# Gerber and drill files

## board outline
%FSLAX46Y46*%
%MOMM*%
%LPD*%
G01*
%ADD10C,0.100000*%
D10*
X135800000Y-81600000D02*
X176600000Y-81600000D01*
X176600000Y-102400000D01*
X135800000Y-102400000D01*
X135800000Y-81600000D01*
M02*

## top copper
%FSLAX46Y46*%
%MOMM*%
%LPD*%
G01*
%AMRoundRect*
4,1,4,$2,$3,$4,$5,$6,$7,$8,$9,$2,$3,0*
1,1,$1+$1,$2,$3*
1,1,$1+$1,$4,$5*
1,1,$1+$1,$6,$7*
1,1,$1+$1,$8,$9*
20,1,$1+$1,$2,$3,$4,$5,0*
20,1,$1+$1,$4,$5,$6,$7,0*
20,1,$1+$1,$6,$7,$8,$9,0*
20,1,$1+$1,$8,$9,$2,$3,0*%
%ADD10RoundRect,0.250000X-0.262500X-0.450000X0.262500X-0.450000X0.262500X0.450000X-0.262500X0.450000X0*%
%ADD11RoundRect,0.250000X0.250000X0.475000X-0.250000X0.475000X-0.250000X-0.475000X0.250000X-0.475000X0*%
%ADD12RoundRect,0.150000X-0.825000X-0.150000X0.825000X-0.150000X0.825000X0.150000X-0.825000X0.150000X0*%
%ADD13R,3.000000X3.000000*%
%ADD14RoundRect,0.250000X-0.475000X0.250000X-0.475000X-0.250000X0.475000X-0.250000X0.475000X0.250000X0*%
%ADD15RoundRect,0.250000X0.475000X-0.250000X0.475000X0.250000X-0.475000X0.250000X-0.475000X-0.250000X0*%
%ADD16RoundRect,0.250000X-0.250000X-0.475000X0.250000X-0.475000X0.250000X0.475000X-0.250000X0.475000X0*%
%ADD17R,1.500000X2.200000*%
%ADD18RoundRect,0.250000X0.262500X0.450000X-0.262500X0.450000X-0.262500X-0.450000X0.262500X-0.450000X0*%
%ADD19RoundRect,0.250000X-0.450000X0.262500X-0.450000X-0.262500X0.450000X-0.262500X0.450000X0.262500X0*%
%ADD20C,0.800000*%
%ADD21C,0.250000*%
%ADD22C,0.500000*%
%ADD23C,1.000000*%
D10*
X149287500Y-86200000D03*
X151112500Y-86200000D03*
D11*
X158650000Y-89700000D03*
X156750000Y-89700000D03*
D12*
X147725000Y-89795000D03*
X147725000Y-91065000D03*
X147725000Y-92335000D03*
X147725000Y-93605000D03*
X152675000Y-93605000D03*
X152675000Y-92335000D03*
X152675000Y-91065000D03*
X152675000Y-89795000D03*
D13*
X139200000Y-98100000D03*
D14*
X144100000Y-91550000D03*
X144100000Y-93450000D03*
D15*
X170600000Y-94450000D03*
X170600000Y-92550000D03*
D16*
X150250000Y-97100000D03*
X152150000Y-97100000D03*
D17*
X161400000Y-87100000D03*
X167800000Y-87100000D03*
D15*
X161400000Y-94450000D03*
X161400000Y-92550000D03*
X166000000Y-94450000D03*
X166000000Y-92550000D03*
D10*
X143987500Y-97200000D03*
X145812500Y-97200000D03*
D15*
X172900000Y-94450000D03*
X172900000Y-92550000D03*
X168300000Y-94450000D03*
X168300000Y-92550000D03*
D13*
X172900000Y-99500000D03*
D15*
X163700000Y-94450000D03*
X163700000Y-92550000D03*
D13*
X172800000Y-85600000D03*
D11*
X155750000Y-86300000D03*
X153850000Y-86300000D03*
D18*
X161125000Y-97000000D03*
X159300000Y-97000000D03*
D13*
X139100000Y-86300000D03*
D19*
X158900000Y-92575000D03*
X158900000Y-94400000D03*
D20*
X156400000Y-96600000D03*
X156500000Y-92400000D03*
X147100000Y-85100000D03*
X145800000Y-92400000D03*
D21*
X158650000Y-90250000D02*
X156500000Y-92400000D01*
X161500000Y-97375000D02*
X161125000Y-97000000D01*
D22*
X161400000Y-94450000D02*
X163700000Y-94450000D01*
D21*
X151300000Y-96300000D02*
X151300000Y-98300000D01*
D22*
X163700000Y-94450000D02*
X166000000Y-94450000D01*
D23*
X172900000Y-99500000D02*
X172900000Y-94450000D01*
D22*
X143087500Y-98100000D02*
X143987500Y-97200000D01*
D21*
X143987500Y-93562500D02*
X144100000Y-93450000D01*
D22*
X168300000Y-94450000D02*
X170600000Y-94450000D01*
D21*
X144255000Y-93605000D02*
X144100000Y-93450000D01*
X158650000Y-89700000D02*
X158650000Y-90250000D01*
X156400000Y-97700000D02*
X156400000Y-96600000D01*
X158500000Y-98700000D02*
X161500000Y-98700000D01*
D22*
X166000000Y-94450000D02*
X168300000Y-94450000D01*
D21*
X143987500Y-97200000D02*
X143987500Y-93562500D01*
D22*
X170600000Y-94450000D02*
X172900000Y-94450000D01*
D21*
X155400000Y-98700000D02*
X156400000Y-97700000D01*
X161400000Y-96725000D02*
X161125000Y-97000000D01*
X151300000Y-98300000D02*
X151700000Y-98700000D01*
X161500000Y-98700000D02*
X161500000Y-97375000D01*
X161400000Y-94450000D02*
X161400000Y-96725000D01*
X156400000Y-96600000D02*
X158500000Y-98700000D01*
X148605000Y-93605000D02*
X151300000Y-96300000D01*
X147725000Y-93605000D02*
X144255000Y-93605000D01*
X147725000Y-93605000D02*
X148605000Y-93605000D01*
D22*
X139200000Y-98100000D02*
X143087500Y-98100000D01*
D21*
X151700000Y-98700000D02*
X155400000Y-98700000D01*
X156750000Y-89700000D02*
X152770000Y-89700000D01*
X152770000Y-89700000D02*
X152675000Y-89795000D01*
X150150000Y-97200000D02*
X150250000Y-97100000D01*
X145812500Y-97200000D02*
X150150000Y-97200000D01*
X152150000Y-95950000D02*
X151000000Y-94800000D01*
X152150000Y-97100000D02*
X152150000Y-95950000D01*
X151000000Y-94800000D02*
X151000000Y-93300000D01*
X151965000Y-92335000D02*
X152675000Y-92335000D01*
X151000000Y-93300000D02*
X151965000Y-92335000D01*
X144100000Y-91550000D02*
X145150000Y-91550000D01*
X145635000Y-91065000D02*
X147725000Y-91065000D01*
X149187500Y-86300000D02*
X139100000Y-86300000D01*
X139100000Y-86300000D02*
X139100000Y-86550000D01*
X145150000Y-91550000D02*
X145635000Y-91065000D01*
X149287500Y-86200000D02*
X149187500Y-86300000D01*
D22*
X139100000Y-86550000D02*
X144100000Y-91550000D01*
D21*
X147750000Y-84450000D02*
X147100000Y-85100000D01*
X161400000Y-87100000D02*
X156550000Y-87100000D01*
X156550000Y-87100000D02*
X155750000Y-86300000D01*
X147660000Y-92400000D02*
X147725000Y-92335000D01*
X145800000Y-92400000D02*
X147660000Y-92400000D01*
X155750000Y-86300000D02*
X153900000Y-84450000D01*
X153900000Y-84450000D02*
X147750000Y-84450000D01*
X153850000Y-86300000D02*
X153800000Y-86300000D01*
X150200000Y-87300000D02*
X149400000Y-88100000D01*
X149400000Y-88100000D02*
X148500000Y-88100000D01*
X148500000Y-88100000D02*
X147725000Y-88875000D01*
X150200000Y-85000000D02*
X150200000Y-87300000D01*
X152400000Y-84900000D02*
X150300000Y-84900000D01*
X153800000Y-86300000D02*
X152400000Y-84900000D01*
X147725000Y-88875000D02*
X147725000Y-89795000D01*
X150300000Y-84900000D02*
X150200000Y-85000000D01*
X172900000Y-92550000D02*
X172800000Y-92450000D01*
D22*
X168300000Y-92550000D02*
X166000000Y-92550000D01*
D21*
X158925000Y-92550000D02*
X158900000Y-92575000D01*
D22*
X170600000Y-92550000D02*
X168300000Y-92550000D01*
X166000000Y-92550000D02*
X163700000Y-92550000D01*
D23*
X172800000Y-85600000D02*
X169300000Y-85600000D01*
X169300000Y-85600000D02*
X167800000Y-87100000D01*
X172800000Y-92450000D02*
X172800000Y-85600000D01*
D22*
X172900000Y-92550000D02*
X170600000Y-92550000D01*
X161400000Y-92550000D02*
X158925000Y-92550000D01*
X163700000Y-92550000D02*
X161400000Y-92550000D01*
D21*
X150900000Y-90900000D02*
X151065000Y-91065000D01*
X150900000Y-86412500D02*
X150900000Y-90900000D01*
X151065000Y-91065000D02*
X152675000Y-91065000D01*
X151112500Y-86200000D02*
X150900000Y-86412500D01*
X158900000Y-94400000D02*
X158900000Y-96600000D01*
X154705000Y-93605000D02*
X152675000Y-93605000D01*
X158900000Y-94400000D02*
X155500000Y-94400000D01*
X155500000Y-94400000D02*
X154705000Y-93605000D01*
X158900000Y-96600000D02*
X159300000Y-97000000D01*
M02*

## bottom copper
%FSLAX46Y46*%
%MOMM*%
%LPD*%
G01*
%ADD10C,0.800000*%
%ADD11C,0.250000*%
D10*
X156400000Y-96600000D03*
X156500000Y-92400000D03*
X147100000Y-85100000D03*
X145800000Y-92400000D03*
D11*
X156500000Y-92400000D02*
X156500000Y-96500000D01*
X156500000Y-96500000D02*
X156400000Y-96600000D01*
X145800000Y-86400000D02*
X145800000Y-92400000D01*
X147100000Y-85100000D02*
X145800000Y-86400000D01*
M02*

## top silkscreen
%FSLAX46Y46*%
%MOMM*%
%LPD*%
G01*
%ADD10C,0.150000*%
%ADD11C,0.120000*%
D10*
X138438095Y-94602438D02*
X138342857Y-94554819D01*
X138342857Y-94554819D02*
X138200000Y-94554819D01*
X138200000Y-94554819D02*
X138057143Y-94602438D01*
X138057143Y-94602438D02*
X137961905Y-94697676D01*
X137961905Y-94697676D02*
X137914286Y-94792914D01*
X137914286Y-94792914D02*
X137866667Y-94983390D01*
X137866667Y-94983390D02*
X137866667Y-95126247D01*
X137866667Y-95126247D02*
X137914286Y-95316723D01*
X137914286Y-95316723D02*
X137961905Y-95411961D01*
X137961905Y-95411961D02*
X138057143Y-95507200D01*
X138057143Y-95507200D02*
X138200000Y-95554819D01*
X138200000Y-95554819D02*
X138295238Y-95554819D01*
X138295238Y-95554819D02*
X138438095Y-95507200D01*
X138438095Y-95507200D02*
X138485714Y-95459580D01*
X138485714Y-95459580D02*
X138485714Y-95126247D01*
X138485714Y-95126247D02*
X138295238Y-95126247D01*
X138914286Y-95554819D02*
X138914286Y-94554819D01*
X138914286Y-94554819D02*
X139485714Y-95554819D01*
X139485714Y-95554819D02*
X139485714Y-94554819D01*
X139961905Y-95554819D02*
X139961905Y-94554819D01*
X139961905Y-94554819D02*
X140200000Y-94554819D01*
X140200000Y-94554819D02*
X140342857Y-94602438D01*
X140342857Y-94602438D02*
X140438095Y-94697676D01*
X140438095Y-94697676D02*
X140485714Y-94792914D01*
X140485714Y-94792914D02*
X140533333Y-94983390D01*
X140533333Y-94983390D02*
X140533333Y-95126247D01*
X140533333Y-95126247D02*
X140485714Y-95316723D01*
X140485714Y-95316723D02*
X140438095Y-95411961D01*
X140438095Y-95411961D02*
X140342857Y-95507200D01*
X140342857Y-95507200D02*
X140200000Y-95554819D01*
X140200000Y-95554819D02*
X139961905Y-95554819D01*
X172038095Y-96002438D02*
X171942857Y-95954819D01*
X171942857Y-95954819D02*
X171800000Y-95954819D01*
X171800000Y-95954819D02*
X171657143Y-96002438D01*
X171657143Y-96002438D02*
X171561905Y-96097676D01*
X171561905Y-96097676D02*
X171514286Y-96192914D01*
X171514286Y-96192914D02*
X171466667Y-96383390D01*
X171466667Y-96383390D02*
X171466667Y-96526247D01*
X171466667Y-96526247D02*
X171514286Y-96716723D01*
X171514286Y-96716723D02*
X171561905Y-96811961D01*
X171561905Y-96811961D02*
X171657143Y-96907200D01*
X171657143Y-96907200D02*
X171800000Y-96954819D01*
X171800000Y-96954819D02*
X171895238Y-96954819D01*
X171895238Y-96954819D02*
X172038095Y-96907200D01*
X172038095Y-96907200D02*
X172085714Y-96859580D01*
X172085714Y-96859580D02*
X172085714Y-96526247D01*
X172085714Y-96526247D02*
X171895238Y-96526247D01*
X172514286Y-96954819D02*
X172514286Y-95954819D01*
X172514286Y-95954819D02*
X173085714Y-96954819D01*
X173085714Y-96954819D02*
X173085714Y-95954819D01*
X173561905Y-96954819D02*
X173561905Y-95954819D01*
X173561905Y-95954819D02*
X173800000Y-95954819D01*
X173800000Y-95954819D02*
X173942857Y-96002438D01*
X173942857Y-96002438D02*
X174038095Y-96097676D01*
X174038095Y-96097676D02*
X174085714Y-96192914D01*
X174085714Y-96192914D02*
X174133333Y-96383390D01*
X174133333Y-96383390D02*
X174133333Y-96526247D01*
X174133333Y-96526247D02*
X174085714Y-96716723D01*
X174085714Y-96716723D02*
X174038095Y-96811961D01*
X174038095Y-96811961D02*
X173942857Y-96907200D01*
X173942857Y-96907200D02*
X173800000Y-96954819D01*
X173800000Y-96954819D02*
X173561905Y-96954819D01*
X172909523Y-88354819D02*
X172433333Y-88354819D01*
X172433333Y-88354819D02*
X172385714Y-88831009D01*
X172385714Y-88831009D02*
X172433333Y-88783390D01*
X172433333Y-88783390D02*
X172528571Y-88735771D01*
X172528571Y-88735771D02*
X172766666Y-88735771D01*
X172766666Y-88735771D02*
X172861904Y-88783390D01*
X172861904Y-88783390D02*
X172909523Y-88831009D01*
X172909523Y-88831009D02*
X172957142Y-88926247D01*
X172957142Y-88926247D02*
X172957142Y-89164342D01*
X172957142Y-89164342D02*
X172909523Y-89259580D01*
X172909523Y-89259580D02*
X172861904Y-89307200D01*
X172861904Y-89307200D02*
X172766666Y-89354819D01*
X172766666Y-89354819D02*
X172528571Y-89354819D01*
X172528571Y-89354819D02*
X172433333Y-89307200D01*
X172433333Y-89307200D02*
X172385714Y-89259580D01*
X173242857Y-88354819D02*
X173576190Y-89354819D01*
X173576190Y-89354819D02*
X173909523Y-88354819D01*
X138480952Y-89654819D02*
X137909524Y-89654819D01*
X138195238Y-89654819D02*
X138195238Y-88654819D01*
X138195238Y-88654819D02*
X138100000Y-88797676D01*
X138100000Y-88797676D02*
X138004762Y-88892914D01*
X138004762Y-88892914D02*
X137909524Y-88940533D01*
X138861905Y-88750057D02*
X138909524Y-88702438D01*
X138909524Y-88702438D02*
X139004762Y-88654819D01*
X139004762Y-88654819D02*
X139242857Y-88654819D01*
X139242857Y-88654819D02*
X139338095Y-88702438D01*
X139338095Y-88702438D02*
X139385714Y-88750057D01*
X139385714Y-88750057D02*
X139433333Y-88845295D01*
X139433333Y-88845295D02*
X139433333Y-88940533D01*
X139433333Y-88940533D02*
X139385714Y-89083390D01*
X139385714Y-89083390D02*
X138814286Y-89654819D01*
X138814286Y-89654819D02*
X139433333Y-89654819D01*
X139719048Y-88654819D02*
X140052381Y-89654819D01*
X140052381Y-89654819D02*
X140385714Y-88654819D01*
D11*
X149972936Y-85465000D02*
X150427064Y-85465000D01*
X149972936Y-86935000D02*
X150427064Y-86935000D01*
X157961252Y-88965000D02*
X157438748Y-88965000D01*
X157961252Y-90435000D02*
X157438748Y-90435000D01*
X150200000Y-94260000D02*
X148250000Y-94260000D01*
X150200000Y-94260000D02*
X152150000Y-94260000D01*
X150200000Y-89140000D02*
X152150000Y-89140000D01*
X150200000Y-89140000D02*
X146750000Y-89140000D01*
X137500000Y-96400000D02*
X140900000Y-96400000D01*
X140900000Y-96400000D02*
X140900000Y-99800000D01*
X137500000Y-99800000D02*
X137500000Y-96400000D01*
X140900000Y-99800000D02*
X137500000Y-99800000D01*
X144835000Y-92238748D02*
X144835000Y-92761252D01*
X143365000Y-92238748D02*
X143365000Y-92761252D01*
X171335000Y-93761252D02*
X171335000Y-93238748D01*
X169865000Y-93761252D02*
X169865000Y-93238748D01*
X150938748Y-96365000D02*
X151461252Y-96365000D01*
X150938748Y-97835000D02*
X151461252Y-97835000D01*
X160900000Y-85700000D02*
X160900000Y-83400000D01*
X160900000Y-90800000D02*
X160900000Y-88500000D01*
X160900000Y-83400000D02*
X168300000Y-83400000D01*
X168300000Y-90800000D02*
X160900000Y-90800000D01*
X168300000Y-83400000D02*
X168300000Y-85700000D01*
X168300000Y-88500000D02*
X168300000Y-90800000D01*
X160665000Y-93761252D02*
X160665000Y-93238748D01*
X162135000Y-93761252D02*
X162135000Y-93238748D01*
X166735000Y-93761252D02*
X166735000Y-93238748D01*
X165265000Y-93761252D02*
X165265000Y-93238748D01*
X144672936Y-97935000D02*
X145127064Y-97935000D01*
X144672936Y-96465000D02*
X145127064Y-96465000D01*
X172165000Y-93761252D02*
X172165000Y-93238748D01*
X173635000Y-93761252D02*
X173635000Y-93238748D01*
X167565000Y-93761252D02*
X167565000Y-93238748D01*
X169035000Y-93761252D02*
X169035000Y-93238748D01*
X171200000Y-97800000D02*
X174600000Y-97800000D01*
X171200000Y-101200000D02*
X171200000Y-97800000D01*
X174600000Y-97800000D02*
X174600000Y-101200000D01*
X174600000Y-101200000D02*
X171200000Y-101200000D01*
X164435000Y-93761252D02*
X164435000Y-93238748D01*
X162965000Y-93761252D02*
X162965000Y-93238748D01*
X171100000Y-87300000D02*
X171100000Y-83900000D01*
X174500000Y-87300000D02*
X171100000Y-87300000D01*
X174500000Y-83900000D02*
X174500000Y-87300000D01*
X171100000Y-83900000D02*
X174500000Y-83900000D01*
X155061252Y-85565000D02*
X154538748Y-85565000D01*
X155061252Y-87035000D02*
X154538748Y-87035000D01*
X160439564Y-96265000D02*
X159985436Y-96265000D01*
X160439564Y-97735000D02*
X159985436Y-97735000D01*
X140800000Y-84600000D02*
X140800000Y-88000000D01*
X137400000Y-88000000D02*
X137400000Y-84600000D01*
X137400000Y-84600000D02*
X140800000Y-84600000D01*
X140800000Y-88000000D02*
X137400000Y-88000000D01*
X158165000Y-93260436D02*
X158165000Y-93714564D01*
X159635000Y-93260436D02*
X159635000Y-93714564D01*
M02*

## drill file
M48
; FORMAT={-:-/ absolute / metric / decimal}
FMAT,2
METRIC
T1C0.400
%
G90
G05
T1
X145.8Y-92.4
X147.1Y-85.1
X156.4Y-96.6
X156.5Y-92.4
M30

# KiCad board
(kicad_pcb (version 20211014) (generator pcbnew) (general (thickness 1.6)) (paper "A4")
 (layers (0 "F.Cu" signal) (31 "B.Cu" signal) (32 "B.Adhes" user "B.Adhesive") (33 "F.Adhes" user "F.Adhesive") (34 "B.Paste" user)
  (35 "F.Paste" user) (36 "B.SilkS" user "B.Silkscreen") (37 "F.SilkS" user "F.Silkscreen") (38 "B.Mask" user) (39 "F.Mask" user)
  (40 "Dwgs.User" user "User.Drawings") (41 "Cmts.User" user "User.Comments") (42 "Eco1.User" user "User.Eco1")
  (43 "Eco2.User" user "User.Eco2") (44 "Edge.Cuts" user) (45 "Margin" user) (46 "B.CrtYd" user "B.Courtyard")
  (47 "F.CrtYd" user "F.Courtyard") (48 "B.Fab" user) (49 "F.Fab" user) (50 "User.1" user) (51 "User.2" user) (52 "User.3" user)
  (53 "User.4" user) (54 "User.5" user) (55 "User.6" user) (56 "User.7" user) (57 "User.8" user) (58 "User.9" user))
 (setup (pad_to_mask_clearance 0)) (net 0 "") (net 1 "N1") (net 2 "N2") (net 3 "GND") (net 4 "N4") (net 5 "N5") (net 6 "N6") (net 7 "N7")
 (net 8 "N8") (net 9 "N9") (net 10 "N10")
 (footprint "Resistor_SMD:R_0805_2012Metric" (layer "F.Cu") (at 150.2 86.2)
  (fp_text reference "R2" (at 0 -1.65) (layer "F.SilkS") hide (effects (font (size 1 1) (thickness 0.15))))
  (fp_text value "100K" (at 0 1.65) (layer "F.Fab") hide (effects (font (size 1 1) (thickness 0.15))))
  (fp_line (start -0.227064 -0.735) (end 0.227064 -0.735) (layer "F.SilkS") (width 0.12))
  (fp_line (start -0.227064 0.735) (end 0.227064 0.735) (layer "F.SilkS") (width 0.12))
  (pad "1" smd roundrect (at -0.9125 0) (size 1.025 1.4) (layers "F.Cu" "F.Paste" "F.Mask") (roundrect_rratio 0.243902439) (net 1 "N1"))
  (pad "2" smd roundrect (at 0.9125 0) (size 1.025 1.4) (layers "F.Cu" "F.Paste" "F.Mask") (roundrect_rratio 0.243902439) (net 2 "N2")))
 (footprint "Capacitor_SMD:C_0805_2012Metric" (layer "F.Cu") (at 157.7 89.7 180)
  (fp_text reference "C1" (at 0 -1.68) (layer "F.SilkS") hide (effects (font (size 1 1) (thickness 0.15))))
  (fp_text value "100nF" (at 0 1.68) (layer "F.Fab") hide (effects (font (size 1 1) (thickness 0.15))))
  (fp_line (start -0.261252 0.735) (end 0.261252 0.735) (layer "F.SilkS") (width 0.12))
  (fp_line (start -0.261252 -0.735) (end 0.261252 -0.735) (layer "F.SilkS") (width 0.12))
  (pad "1" smd roundrect (at -0.95 0 180) (size 1 1.45) (layers "F.Cu" "F.Paste" "F.Mask") (roundrect_rratio 0.25) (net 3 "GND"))
  (pad "2" smd roundrect (at 0.95 0 180) (size 1 1.45) (layers "F.Cu" "F.Paste" "F.Mask") (roundrect_rratio 0.25) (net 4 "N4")))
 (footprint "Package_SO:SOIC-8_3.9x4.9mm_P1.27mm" (layer "F.Cu") (at 150.2 91.7)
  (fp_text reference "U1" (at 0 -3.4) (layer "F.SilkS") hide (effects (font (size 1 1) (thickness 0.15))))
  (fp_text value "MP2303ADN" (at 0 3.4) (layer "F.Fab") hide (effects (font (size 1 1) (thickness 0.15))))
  (fp_line (start 0 2.56) (end -1.95 2.56) (layer "F.SilkS") (width 0.12))
  (fp_line (start 0 2.56) (end 1.95 2.56) (layer "F.SilkS") (width 0.12))
  (fp_line (start 0 -2.56) (end 1.95 -2.56) (layer "F.SilkS") (width 0.12))
  (fp_line (start 0 -2.56) (end -3.45 -2.56) (layer "F.SilkS") (width 0.12))
  (pad "1" smd roundrect (at -2.475 -1.905) (size 1.95 0.6) (layers "F.Cu" "F.Paste" "F.Mask") (roundrect_rratio 0.25) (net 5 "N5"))
  (pad "2" smd roundrect (at -2.475 -0.635) (size 1.95 0.6) (layers "F.Cu" "F.Paste" "F.Mask") (roundrect_rratio 0.25) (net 1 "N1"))
  (pad "3" smd roundrect (at -2.475 0.635) (size 1.95 0.6) (layers "F.Cu" "F.Paste" "F.Mask") (roundrect_rratio 0.25) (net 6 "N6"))
  (pad "4" smd roundrect (at -2.475 1.905) (size 1.95 0.6) (layers "F.Cu" "F.Paste" "F.Mask") (roundrect_rratio 0.25) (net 3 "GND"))
  (pad "5" smd roundrect (at 2.475 1.905) (size 1.95 0.6) (layers "F.Cu" "F.Paste" "F.Mask") (roundrect_rratio 0.25) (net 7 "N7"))
  (pad "6" smd roundrect (at 2.475 0.635) (size 1.95 0.6) (layers "F.Cu" "F.Paste" "F.Mask") (roundrect_rratio 0.25) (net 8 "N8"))
  (pad "7" smd roundrect (at 2.475 -0.635) (size 1.95 0.6) (layers "F.Cu" "F.Paste" "F.Mask") (roundrect_rratio 0.25) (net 2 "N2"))
  (pad "8" smd roundrect (at 2.475 -1.905) (size 1.95 0.6) (layers "F.Cu" "F.Paste" "F.Mask") (roundrect_rratio 0.25) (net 4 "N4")))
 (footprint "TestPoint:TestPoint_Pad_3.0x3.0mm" (layer "F.Cu") (at 139.2 98.1)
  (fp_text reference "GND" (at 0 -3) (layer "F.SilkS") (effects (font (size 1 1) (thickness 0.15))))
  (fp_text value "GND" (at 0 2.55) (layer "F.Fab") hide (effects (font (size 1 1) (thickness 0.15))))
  (fp_line (start -1.7 -1.7) (end 1.7 -1.7) (layer "F.SilkS") (width 0.12))
  (fp_line (start 1.7 -1.7) (end 1.7 1.7) (layer "F.SilkS") (width 0.12))
  (fp_line (start -1.7 1.7) (end -1.7 -1.7) (layer "F.SilkS") (width 0.12))
  (fp_line (start 1.7 1.7) (end -1.7 1.7) (layer "F.SilkS") (width 0.12))
  (pad "1" smd rect (at 0 0) (size 3 3) (layers "F.Cu" "F.Mask") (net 3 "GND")))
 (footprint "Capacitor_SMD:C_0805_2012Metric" (layer "F.Cu") (at 144.1 92.5 -90)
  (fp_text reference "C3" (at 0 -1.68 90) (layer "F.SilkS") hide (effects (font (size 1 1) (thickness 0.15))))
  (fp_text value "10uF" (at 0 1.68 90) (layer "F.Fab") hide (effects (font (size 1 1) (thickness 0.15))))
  (fp_line (start -0.261252 -0.735) (end 0.261252 -0.735) (layer "F.SilkS") (width 0.12))
  (fp_line (start -0.261252 0.735) (end 0.261252 0.735) (layer "F.SilkS") (width 0.12))
  (pad "1" smd roundrect (at -0.95 0 270) (size 1 1.45) (layers "F.Cu" "F.Paste" "F.Mask") (roundrect_rratio 0.25) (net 1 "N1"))
  (pad "2" smd roundrect (at 0.95 0 270) (size 1 1.45) (layers "F.Cu" "F.Paste" "F.Mask") (roundrect_rratio 0.25) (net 3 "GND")))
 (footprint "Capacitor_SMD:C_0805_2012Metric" (layer "F.Cu") (at 170.6 93.5 90)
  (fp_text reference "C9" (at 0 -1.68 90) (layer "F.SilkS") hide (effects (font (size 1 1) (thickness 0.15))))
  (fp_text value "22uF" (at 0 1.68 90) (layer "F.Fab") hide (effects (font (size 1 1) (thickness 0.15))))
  (fp_line (start -0.261252 0.735) (end 0.261252 0.735) (layer "F.SilkS") (width 0.12))
  (fp_line (start -0.261252 -0.735) (end 0.261252 -0.735) (layer "F.SilkS") (width 0.12))
  (pad "1" smd roundrect (at -0.95 0 90) (size 1 1.45) (layers "F.Cu" "F.Paste" "F.Mask") (roundrect_rratio 0.25) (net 3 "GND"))
  (pad "2" smd roundrect (at 0.95 0 90) (size 1 1.45) (layers "F.Cu" "F.Paste" "F.Mask") (roundrect_rratio 0.25) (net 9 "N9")))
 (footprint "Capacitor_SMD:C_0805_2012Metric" (layer "F.Cu") (at 151.2 97.1)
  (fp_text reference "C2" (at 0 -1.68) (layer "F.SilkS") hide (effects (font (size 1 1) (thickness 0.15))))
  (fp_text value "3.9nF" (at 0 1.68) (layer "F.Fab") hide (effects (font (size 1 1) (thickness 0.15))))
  (fp_line (start -0.261252 -0.735) (end 0.261252 -0.735) (layer "F.SilkS") (width 0.12))
  (fp_line (start -0.261252 0.735) (end 0.261252 0.735) (layer "F.SilkS") (width 0.12))
  (pad "1" smd roundrect (at -0.95 0) (size 1 1.45) (layers "F.Cu" "F.Paste" "F.Mask") (roundrect_rratio 0.25) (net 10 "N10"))
  (pad "2" smd roundrect (at 0.95 0) (size 1 1.45) (layers "F.Cu" "F.Paste" "F.Mask") (roundrect_rratio 0.25) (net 8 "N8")))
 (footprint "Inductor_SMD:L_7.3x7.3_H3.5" (layer "F.Cu") (at 164.6 87.1)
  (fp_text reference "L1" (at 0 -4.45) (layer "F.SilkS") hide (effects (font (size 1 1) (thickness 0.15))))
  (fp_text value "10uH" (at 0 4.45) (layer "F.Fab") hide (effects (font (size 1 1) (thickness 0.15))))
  (fp_line (start -3.7 -1.4) (end -3.7 -3.7) (layer "F.SilkS") (width 0.12))
  (fp_line (start -3.7 3.7) (end -3.7 1.4) (layer "F.SilkS") (width 0.12))
  (fp_line (start -3.7 -3.7) (end 3.7 -3.7) (layer "F.SilkS") (width 0.12))
  (fp_line (start 3.7 3.7) (end -3.7 3.7) (layer "F.SilkS") (width 0.12))
  (fp_line (start 3.7 -3.7) (end 3.7 -1.4) (layer "F.SilkS") (width 0.12))
  (fp_line (start 3.7 1.4) (end 3.7 3.7) (layer "F.SilkS") (width 0.12))
  (pad "1" smd rect (at -3.2 0) (size 1.5 2.2) (layers "F.Cu" "F.Paste" "F.Mask") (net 6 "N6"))
  (pad "2" smd rect (at 3.2 0) (size 1.5 2.2) (layers "F.Cu" "F.Paste" "F.Mask") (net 9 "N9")))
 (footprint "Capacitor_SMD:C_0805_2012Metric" (layer "F.Cu") (at 161.4 93.5 90)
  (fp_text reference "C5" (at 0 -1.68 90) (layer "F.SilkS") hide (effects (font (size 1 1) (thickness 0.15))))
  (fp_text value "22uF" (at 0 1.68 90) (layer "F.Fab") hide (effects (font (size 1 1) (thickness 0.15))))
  (fp_line (start -0.261252 -0.735) (end 0.261252 -0.735) (layer "F.SilkS") (width 0.12))
  (fp_line (start -0.261252 0.735) (end 0.261252 0.735) (layer "F.SilkS") (width 0.12))
  (pad "1" smd roundrect (at -0.95 0 90) (size 1 1.45) (layers "F.Cu" "F.Paste" "F.Mask") (roundrect_rratio 0.25) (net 3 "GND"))
  (pad "2" smd roundrect (at 0.95 0 90) (size 1 1.45) (layers "F.Cu" "F.Paste" "F.Mask") (roundrect_rratio 0.25) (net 9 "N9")))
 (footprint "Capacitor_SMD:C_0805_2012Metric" (layer "F.Cu") (at 166 93.5 90)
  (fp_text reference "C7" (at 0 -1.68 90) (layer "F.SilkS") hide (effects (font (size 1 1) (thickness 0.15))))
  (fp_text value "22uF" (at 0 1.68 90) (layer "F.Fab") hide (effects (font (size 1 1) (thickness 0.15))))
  (fp_line (start -0.261252 0.735) (end 0.261252 0.735) (layer "F.SilkS") (width 0.12))
  (fp_line (start -0.261252 -0.735) (end 0.261252 -0.735) (layer "F.SilkS") (width 0.12))
  (pad "1" smd roundrect (at -0.95 0 90) (size 1 1.45) (layers "F.Cu" "F.Paste" "F.Mask") (roundrect_rratio 0.25) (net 3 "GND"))
  (pad "2" smd roundrect (at 0.95 0 90) (size 1 1.45) (layers "F.Cu" "F.Paste" "F.Mask") (roundrect_rratio 0.25) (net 9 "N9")))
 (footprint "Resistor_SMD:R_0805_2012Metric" (layer "F.Cu") (at 144.9 97.2)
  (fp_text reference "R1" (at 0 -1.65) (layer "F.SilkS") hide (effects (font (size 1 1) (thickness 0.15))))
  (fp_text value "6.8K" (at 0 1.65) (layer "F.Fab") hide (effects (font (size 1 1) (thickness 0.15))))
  (fp_line (start -0.227064 0.735) (end 0.227064 0.735) (layer "F.SilkS") (width 0.12))
  (fp_line (start -0.227064 -0.735) (end 0.227064 -0.735) (layer "F.SilkS") (width 0.12))
  (pad "1" smd roundrect (at -0.9125 0) (size 1.025 1.4) (layers "F.Cu" "F.Paste" "F.Mask") (roundrect_rratio 0.243902439) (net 3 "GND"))
  (pad "2" smd roundrect (at 0.9125 0) (size 1.025 1.4) (layers "F.Cu" "F.Paste" "F.Mask") (roundrect_rratio 0.243902439) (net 10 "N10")))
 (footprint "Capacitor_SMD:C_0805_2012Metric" (layer "F.Cu") (at 172.9 93.5 90)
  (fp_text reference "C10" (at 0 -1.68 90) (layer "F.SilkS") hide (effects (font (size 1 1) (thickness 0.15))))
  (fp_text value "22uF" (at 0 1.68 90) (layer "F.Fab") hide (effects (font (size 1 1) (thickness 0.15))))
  (fp_line (start -0.261252 -0.735) (end 0.261252 -0.735) (layer "F.SilkS") (width 0.12))
  (fp_line (start -0.261252 0.735) (end 0.261252 0.735) (layer "F.SilkS") (width 0.12))
  (pad "1" smd roundrect (at -0.95 0 90) (size 1 1.45) (layers "F.Cu" "F.Paste" "F.Mask") (roundrect_rratio 0.25) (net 3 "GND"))
  (pad "2" smd roundrect (at 0.95 0 90) (size 1 1.45) (layers "F.Cu" "F.Paste" "F.Mask") (roundrect_rratio 0.25) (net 9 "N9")))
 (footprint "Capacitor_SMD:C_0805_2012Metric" (layer "F.Cu") (at 168.3 93.5 90)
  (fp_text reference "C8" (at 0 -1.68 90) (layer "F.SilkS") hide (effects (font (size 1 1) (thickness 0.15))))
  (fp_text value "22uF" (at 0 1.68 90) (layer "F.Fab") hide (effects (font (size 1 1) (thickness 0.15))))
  (fp_line (start -0.261252 -0.735) (end 0.261252 -0.735) (layer "F.SilkS") (width 0.12))
  (fp_line (start -0.261252 0.735) (end 0.261252 0.735) (layer "F.SilkS") (width 0.12))
  (pad "1" smd roundrect (at -0.95 0 90) (size 1 1.45) (layers "F.Cu" "F.Paste" "F.Mask") (roundrect_rratio 0.25) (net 3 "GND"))
  (pad "2" smd roundrect (at 0.95 0 90) (size 1 1.45) (layers "F.Cu" "F.Paste" "F.Mask") (roundrect_rratio 0.25) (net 9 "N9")))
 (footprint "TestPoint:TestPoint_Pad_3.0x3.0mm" (layer "F.Cu") (at 172.9 99.5)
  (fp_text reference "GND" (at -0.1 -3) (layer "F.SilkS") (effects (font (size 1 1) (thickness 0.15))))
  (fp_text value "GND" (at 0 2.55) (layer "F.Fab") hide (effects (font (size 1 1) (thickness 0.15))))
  (fp_line (start -1.7 -1.7) (end 1.7 -1.7) (layer "F.SilkS") (width 0.12))
  (fp_line (start -1.7 1.7) (end -1.7 -1.7) (layer "F.SilkS") (width 0.12))
  (fp_line (start 1.7 -1.7) (end 1.7 1.7) (layer "F.SilkS") (width 0.12))
  (fp_line (start 1.7 1.7) (end -1.7 1.7) (layer "F.SilkS") (width 0.12))
  (pad "1" smd rect (at 0 0) (size 3 3) (layers "F.Cu" "F.Mask") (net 3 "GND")))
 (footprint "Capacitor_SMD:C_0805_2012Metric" (layer "F.Cu") (at 163.7 93.5 90)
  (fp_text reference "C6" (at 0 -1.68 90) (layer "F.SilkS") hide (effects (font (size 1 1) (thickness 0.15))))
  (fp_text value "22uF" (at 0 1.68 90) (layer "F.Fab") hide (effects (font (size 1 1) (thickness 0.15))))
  (fp_line (start -0.261252 0.735) (end 0.261252 0.735) (layer "F.SilkS") (width 0.12))
  (fp_line (start -0.261252 -0.735) (end 0.261252 -0.735) (layer "F.SilkS") (width 0.12))
  (pad "1" smd roundrect (at -0.95 0 90) (size 1 1.45) (layers "F.Cu" "F.Paste" "F.Mask") (roundrect_rratio 0.25) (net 3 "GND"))
  (pad "2" smd roundrect (at 0.95 0 90) (size 1 1.45) (layers "F.Cu" "F.Paste" "F.Mask") (roundrect_rratio 0.25) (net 9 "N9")))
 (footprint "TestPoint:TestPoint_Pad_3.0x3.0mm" (layer "F.Cu") (at 172.8 85.6 180)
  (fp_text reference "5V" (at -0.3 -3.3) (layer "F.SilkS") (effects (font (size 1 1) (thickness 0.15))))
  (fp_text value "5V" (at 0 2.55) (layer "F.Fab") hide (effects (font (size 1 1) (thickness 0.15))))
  (fp_line (start 1.7 -1.7) (end 1.7 1.7) (layer "F.SilkS") (width 0.12))
  (fp_line (start -1.7 -1.7) (end 1.7 -1.7) (layer "F.SilkS") (width 0.12))
  (fp_line (start -1.7 1.7) (end -1.7 -1.7) (layer "F.SilkS") (width 0.12))
  (fp_line (start 1.7 1.7) (end -1.7 1.7) (layer "F.SilkS") (width 0.12))
  (pad "1" smd rect (at 0 0 180) (size 3 3) (layers "F.Cu" "F.Mask") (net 9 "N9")))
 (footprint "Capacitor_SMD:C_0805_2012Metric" (layer "F.Cu") (at 154.8 86.3 180)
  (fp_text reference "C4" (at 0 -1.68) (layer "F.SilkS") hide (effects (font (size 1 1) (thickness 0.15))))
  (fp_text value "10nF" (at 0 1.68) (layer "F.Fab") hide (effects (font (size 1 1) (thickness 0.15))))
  (fp_line (start -0.261252 0.735) (end 0.261252 0.735) (layer "F.SilkS") (width 0.12))
  (fp_line (start -0.261252 -0.735) (end 0.261252 -0.735) (layer "F.SilkS") (width 0.12))
  (pad "1" smd roundrect (at -0.95 0 180) (size 1 1.45) (layers "F.Cu" "F.Paste" "F.Mask") (roundrect_rratio 0.25) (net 6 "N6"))
  (pad "2" smd roundrect (at 0.95 0 180) (size 1 1.45) (layers "F.Cu" "F.Paste" "F.Mask") (roundrect_rratio 0.25) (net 5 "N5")))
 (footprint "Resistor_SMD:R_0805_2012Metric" (layer "F.Cu") (at 160.2125 97 180)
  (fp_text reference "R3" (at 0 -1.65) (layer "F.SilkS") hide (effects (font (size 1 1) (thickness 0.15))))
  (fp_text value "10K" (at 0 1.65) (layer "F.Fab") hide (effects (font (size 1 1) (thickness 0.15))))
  (fp_line (start -0.227064 0.735) (end 0.227064 0.735) (layer "F.SilkS") (width 0.12))
  (fp_line (start -0.227064 -0.735) (end 0.227064 -0.735) (layer "F.SilkS") (width 0.12))
  (pad "1" smd roundrect (at -0.9125 0 180) (size 1.025 1.4) (layers "F.Cu" "F.Paste" "F.Mask") (roundrect_rratio 0.243902439) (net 3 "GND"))
  (pad "2" smd roundrect (at 0.9125 0 180) (size 1.025 1.4) (layers "F.Cu" "F.Paste" "F.Mask") (roundrect_rratio 0.243902439) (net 7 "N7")))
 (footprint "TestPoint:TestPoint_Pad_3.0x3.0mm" (layer "F.Cu") (at 139.1 86.3)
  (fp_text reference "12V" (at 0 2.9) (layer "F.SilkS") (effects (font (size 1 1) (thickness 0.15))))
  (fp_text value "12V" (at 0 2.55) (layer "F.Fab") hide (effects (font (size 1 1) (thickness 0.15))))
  (fp_line (start 1.7 -1.7) (end 1.7 1.7) (layer "F.SilkS") (width 0.12))
  (fp_line (start -1.7 1.7) (end -1.7 -1.7) (layer "F.SilkS") (width 0.12))
  (fp_line (start -1.7 -1.7) (end 1.7 -1.7) (layer "F.SilkS") (width 0.12))
  (fp_line (start 1.7 1.7) (end -1.7 1.7) (layer "F.SilkS") (width 0.12))
  (pad "1" smd rect (at 0 0) (size 3 3) (layers "F.Cu" "F.Mask") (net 1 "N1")))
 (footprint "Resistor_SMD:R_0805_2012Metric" (layer "F.Cu") (at 158.9 93.4875 -90)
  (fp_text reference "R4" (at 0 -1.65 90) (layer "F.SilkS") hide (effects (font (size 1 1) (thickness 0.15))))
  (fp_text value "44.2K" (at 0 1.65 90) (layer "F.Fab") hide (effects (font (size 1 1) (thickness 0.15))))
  (fp_line (start -0.227064 0.735) (end 0.227064 0.735) (layer "F.SilkS") (width 0.12))
  (fp_line (start -0.227064 -0.735) (end 0.227064 -0.735) (layer "F.SilkS") (width 0.12))
  (pad "1" smd roundrect (at -0.9125 0 270) (size 1.025 1.4) (layers "F.Cu" "F.Paste" "F.Mask") (roundrect_rratio 0.243902439) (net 9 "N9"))
  (pad "2" smd roundrect (at 0.9125 0 270) (size 1.025 1.4) (layers "F.Cu" "F.Paste" "F.Mask") (roundrect_rratio 0.243902439) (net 7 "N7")))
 (gr_rect (start 135.8 81.6) (end 176.6 102.4) (layer "Edge.Cuts") (width 0.1) (fill none))
 (segment (start 158.65 90.25) (end 156.5 92.4) (width 0.25) (layer "F.Cu") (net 3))
 (segment (start 161.5 97.375) (end 161.125 97) (width 0.25) (layer "F.Cu") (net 3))
 (segment (start 161.4 94.45) (end 163.7 94.45) (width 0.5) (layer "F.Cu") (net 3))
 (segment (start 151.3 96.3) (end 151.3 98.3) (width 0.25) (layer "F.Cu") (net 3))
 (segment (start 163.7 94.45) (end 166 94.45) (width 0.5) (layer "F.Cu") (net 3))
 (segment (start 172.9 99.5) (end 172.9 94.45) (width 1) (layer "F.Cu") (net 3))
 (segment (start 143.0875 98.1) (end 143.9875 97.2) (width 0.5) (layer "F.Cu") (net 3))
 (segment (start 143.9875 93.5625) (end 144.1 93.45) (width 0.25) (layer "F.Cu") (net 3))
 (segment (start 168.3 94.45) (end 170.6 94.45) (width 0.5) (layer "F.Cu") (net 3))
 (segment (start 144.255 93.605) (end 144.1 93.45) (width 0.25) (layer "F.Cu") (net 3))
 (segment (start 158.65 89.7) (end 158.65 90.25) (width 0.25) (layer "F.Cu") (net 3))
 (segment (start 156.4 97.7) (end 156.4 96.6) (width 0.25) (layer "F.Cu") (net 3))
 (segment (start 158.5 98.7) (end 161.5 98.7) (width 0.25) (layer "F.Cu") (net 3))
 (segment (start 166 94.45) (end 168.3 94.45) (width 0.5) (layer "F.Cu") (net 3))
 (segment (start 143.9875 97.2) (end 143.9875 93.5625) (width 0.25) (layer "F.Cu") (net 3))
 (segment (start 170.6 94.45) (end 172.9 94.45) (width 0.5) (layer "F.Cu") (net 3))
 (segment (start 155.4 98.7) (end 156.4 97.7) (width 0.25) (layer "F.Cu") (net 3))
 (segment (start 161.4 96.725) (end 161.125 97) (width 0.25) (layer "F.Cu") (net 3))
 (segment (start 151.3 98.3) (end 151.7 98.7) (width 0.25) (layer "F.Cu") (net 3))
 (segment (start 161.5 98.7) (end 161.5 97.375) (width 0.25) (layer "F.Cu") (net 3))
 (segment (start 161.4 94.45) (end 161.4 96.725) (width 0.25) (layer "F.Cu") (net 3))
 (segment (start 156.4 96.6) (end 158.5 98.7) (width 0.25) (layer "F.Cu") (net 3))
 (segment (start 148.605 93.605) (end 151.3 96.3) (width 0.25) (layer "F.Cu") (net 3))
 (segment (start 147.725 93.605) (end 144.255 93.605) (width 0.25) (layer "F.Cu") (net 3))
 (segment (start 147.725 93.605) (end 148.605 93.605) (width 0.25) (layer "F.Cu") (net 3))
 (segment (start 139.2 98.1) (end 143.0875 98.1) (width 0.5) (layer "F.Cu") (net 3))
 (segment (start 151.7 98.7) (end 155.4 98.7) (width 0.25) (layer "F.Cu") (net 3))
 (via (at 156.4 96.6) (size 0.8) (drill 0.4) (layers "F.Cu" "B.Cu") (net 3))
 (via (at 156.5 92.4) (size 0.8) (drill 0.4) (layers "F.Cu" "B.Cu") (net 3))
 (segment (start 156.5 92.4) (end 156.5 96.5) (width 0.25) (layer "B.Cu") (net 3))
 (segment (start 156.5 96.5) (end 156.4 96.6) (width 0.25) (layer "B.Cu") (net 3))
 (segment (start 156.75 89.7) (end 152.77 89.7) (width 0.25) (layer "F.Cu") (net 4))
 (segment (start 152.77 89.7) (end 152.675 89.795) (width 0.25) (layer "F.Cu") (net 4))
 (segment (start 150.15 97.2) (end 150.25 97.1) (width 0.25) (layer "F.Cu") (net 10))
 (segment (start 145.8125 97.2) (end 150.15 97.2) (width 0.25) (layer "F.Cu") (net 10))
 (segment (start 152.15 95.95) (end 151 94.8) (width 0.25) (layer "F.Cu") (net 8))
 (segment (start 152.15 97.1) (end 152.15 95.95) (width 0.25) (layer "F.Cu") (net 8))
 (segment (start 151 94.8) (end 151 93.3) (width 0.25) (layer "F.Cu") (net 8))
 (segment (start 151.965 92.335) (end 152.675 92.335) (width 0.25) (layer "F.Cu") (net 8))
 (segment (start 151 93.3) (end 151.965 92.335) (width 0.25) (layer "F.Cu") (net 8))
 (segment (start 144.1 91.55) (end 145.15 91.55) (width 0.25) (layer "F.Cu") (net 1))
 (segment (start 145.635 91.065) (end 147.725 91.065) (width 0.25) (layer "F.Cu") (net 1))
 (segment (start 149.1875 86.3) (end 139.1 86.3) (width 0.25) (layer "F.Cu") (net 1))
 (segment (start 139.1 86.3) (end 139.1 86.55) (width 0.25) (layer "F.Cu") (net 1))
 (segment (start 145.15 91.55) (end 145.635 91.065) (width 0.25) (layer "F.Cu") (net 1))
 (segment (start 149.2875 86.2) (end 149.1875 86.3) (width 0.25) (layer "F.Cu") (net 1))
 (segment (start 139.1 86.55) (end 144.1 91.55) (width 0.5) (layer "F.Cu") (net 1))
 (segment (start 147.75 84.45) (end 147.1 85.1) (width 0.25) (layer "F.Cu") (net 6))
 (segment (start 161.4 87.1) (end 156.55 87.1) (width 0.25) (layer "F.Cu") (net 6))
 (segment (start 156.55 87.1) (end 155.75 86.3) (width 0.25) (layer "F.Cu") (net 6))
 (segment (start 147.66 92.4) (end 147.725 92.335) (width 0.25) (layer "F.Cu") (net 6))
 (segment (start 145.8 92.4) (end 147.66 92.4) (width 0.25) (layer "F.Cu") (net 6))
 (segment (start 155.75 86.3) (end 153.9 84.45) (width 0.25) (layer "F.Cu") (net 6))
 (segment (start 153.9 84.45) (end 147.75 84.45) (width 0.25) (layer "F.Cu") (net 6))
 (via (at 147.1 85.1) (size 0.8) (drill 0.4) (layers "F.Cu" "B.Cu") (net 6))
 (via (at 145.8 92.4) (size 0.8) (drill 0.4) (layers "F.Cu" "B.Cu") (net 6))
 (segment (start 145.8 86.4) (end 145.8 92.4) (width 0.25) (layer "B.Cu") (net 6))
 (segment (start 147.1 85.1) (end 145.8 86.4) (width 0.25) (layer "B.Cu") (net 6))
 (segment (start 153.85 86.3) (end 153.8 86.3) (width 0.25) (layer "F.Cu") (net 5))
 (segment (start 150.2 87.3) (end 149.4 88.1) (width 0.25) (layer "F.Cu") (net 5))
 (segment (start 149.4 88.1) (end 148.5 88.1) (width 0.25) (layer "F.Cu") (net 5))
 (segment (start 148.5 88.1) (end 147.725 88.875) (width 0.25) (layer "F.Cu") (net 5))
 (segment (start 150.2 85) (end 150.2 87.3) (width 0.25) (layer "F.Cu") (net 5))
 (segment (start 152.4 84.9) (end 150.3 84.9) (width 0.25) (layer "F.Cu") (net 5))
 (segment (start 153.8 86.3) (end 152.4 84.9) (width 0.25) (layer "F.Cu") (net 5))
 (segment (start 147.725 88.875) (end 147.725 89.795) (width 0.25) (layer "F.Cu") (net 5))
 (segment (start 150.3 84.9) (end 150.2 85) (width 0.25) (layer "F.Cu") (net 5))
 (segment (start 172.9 92.55) (end 172.8 92.45) (width 0.25) (layer "F.Cu") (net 9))
 (segment (start 168.3 92.55) (end 166 92.55) (width 0.5) (layer "F.Cu") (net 9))
 (segment (start 158.925 92.55) (end 158.9 92.575) (width 0.25) (layer "F.Cu") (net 9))
 (segment (start 170.6 92.55) (end 168.3 92.55) (width 0.5) (layer "F.Cu") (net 9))
 (segment (start 166 92.55) (end 163.7 92.55) (width 0.5) (layer "F.Cu") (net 9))
 (segment (start 172.8 85.6) (end 169.3 85.6) (width 1) (layer "F.Cu") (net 9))
 (segment (start 169.3 85.6) (end 167.8 87.1) (width 1) (layer "F.Cu") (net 9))
 (segment (start 172.8 92.45) (end 172.8 85.6) (width 1) (layer "F.Cu") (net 9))
 (segment (start 172.9 92.55) (end 170.6 92.55) (width 0.5) (layer "F.Cu") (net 9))
 (segment (start 161.4 92.55) (end 158.925 92.55) (width 0.5) (layer "F.Cu") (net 9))
 (segment (start 163.7 92.55) (end 161.4 92.55) (width 0.5) (layer "F.Cu") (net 9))
 (segment (start 150.9 90.9) (end 151.065 91.065) (width 0.25) (layer "F.Cu") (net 2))
 (segment (start 150.9 86.4125) (end 150.9 90.9) (width 0.25) (layer "F.Cu") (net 2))
 (segment (start 151.065 91.065) (end 152.675 91.065) (width 0.25) (layer "F.Cu") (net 2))
 (segment (start 151.1125 86.2) (end 150.9 86.4125) (width 0.25) (layer "F.Cu") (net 2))
 (segment (start 158.9 94.4) (end 158.9 96.6) (width 0.25) (layer "F.Cu") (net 7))
 (segment (start 154.705 93.605) (end 152.675 93.605) (width 0.25) (layer "F.Cu") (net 7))
 (segment (start 158.9 94.4) (end 155.5 94.4) (width 0.25) (layer "F.Cu") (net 7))
 (segment (start 155.5 94.4) (end 154.705 93.605) (width 0.25) (layer "F.Cu") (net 7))
 (segment (start 158.9 96.6) (end 159.3 97) (width 0.25) (layer "F.Cu") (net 7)))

